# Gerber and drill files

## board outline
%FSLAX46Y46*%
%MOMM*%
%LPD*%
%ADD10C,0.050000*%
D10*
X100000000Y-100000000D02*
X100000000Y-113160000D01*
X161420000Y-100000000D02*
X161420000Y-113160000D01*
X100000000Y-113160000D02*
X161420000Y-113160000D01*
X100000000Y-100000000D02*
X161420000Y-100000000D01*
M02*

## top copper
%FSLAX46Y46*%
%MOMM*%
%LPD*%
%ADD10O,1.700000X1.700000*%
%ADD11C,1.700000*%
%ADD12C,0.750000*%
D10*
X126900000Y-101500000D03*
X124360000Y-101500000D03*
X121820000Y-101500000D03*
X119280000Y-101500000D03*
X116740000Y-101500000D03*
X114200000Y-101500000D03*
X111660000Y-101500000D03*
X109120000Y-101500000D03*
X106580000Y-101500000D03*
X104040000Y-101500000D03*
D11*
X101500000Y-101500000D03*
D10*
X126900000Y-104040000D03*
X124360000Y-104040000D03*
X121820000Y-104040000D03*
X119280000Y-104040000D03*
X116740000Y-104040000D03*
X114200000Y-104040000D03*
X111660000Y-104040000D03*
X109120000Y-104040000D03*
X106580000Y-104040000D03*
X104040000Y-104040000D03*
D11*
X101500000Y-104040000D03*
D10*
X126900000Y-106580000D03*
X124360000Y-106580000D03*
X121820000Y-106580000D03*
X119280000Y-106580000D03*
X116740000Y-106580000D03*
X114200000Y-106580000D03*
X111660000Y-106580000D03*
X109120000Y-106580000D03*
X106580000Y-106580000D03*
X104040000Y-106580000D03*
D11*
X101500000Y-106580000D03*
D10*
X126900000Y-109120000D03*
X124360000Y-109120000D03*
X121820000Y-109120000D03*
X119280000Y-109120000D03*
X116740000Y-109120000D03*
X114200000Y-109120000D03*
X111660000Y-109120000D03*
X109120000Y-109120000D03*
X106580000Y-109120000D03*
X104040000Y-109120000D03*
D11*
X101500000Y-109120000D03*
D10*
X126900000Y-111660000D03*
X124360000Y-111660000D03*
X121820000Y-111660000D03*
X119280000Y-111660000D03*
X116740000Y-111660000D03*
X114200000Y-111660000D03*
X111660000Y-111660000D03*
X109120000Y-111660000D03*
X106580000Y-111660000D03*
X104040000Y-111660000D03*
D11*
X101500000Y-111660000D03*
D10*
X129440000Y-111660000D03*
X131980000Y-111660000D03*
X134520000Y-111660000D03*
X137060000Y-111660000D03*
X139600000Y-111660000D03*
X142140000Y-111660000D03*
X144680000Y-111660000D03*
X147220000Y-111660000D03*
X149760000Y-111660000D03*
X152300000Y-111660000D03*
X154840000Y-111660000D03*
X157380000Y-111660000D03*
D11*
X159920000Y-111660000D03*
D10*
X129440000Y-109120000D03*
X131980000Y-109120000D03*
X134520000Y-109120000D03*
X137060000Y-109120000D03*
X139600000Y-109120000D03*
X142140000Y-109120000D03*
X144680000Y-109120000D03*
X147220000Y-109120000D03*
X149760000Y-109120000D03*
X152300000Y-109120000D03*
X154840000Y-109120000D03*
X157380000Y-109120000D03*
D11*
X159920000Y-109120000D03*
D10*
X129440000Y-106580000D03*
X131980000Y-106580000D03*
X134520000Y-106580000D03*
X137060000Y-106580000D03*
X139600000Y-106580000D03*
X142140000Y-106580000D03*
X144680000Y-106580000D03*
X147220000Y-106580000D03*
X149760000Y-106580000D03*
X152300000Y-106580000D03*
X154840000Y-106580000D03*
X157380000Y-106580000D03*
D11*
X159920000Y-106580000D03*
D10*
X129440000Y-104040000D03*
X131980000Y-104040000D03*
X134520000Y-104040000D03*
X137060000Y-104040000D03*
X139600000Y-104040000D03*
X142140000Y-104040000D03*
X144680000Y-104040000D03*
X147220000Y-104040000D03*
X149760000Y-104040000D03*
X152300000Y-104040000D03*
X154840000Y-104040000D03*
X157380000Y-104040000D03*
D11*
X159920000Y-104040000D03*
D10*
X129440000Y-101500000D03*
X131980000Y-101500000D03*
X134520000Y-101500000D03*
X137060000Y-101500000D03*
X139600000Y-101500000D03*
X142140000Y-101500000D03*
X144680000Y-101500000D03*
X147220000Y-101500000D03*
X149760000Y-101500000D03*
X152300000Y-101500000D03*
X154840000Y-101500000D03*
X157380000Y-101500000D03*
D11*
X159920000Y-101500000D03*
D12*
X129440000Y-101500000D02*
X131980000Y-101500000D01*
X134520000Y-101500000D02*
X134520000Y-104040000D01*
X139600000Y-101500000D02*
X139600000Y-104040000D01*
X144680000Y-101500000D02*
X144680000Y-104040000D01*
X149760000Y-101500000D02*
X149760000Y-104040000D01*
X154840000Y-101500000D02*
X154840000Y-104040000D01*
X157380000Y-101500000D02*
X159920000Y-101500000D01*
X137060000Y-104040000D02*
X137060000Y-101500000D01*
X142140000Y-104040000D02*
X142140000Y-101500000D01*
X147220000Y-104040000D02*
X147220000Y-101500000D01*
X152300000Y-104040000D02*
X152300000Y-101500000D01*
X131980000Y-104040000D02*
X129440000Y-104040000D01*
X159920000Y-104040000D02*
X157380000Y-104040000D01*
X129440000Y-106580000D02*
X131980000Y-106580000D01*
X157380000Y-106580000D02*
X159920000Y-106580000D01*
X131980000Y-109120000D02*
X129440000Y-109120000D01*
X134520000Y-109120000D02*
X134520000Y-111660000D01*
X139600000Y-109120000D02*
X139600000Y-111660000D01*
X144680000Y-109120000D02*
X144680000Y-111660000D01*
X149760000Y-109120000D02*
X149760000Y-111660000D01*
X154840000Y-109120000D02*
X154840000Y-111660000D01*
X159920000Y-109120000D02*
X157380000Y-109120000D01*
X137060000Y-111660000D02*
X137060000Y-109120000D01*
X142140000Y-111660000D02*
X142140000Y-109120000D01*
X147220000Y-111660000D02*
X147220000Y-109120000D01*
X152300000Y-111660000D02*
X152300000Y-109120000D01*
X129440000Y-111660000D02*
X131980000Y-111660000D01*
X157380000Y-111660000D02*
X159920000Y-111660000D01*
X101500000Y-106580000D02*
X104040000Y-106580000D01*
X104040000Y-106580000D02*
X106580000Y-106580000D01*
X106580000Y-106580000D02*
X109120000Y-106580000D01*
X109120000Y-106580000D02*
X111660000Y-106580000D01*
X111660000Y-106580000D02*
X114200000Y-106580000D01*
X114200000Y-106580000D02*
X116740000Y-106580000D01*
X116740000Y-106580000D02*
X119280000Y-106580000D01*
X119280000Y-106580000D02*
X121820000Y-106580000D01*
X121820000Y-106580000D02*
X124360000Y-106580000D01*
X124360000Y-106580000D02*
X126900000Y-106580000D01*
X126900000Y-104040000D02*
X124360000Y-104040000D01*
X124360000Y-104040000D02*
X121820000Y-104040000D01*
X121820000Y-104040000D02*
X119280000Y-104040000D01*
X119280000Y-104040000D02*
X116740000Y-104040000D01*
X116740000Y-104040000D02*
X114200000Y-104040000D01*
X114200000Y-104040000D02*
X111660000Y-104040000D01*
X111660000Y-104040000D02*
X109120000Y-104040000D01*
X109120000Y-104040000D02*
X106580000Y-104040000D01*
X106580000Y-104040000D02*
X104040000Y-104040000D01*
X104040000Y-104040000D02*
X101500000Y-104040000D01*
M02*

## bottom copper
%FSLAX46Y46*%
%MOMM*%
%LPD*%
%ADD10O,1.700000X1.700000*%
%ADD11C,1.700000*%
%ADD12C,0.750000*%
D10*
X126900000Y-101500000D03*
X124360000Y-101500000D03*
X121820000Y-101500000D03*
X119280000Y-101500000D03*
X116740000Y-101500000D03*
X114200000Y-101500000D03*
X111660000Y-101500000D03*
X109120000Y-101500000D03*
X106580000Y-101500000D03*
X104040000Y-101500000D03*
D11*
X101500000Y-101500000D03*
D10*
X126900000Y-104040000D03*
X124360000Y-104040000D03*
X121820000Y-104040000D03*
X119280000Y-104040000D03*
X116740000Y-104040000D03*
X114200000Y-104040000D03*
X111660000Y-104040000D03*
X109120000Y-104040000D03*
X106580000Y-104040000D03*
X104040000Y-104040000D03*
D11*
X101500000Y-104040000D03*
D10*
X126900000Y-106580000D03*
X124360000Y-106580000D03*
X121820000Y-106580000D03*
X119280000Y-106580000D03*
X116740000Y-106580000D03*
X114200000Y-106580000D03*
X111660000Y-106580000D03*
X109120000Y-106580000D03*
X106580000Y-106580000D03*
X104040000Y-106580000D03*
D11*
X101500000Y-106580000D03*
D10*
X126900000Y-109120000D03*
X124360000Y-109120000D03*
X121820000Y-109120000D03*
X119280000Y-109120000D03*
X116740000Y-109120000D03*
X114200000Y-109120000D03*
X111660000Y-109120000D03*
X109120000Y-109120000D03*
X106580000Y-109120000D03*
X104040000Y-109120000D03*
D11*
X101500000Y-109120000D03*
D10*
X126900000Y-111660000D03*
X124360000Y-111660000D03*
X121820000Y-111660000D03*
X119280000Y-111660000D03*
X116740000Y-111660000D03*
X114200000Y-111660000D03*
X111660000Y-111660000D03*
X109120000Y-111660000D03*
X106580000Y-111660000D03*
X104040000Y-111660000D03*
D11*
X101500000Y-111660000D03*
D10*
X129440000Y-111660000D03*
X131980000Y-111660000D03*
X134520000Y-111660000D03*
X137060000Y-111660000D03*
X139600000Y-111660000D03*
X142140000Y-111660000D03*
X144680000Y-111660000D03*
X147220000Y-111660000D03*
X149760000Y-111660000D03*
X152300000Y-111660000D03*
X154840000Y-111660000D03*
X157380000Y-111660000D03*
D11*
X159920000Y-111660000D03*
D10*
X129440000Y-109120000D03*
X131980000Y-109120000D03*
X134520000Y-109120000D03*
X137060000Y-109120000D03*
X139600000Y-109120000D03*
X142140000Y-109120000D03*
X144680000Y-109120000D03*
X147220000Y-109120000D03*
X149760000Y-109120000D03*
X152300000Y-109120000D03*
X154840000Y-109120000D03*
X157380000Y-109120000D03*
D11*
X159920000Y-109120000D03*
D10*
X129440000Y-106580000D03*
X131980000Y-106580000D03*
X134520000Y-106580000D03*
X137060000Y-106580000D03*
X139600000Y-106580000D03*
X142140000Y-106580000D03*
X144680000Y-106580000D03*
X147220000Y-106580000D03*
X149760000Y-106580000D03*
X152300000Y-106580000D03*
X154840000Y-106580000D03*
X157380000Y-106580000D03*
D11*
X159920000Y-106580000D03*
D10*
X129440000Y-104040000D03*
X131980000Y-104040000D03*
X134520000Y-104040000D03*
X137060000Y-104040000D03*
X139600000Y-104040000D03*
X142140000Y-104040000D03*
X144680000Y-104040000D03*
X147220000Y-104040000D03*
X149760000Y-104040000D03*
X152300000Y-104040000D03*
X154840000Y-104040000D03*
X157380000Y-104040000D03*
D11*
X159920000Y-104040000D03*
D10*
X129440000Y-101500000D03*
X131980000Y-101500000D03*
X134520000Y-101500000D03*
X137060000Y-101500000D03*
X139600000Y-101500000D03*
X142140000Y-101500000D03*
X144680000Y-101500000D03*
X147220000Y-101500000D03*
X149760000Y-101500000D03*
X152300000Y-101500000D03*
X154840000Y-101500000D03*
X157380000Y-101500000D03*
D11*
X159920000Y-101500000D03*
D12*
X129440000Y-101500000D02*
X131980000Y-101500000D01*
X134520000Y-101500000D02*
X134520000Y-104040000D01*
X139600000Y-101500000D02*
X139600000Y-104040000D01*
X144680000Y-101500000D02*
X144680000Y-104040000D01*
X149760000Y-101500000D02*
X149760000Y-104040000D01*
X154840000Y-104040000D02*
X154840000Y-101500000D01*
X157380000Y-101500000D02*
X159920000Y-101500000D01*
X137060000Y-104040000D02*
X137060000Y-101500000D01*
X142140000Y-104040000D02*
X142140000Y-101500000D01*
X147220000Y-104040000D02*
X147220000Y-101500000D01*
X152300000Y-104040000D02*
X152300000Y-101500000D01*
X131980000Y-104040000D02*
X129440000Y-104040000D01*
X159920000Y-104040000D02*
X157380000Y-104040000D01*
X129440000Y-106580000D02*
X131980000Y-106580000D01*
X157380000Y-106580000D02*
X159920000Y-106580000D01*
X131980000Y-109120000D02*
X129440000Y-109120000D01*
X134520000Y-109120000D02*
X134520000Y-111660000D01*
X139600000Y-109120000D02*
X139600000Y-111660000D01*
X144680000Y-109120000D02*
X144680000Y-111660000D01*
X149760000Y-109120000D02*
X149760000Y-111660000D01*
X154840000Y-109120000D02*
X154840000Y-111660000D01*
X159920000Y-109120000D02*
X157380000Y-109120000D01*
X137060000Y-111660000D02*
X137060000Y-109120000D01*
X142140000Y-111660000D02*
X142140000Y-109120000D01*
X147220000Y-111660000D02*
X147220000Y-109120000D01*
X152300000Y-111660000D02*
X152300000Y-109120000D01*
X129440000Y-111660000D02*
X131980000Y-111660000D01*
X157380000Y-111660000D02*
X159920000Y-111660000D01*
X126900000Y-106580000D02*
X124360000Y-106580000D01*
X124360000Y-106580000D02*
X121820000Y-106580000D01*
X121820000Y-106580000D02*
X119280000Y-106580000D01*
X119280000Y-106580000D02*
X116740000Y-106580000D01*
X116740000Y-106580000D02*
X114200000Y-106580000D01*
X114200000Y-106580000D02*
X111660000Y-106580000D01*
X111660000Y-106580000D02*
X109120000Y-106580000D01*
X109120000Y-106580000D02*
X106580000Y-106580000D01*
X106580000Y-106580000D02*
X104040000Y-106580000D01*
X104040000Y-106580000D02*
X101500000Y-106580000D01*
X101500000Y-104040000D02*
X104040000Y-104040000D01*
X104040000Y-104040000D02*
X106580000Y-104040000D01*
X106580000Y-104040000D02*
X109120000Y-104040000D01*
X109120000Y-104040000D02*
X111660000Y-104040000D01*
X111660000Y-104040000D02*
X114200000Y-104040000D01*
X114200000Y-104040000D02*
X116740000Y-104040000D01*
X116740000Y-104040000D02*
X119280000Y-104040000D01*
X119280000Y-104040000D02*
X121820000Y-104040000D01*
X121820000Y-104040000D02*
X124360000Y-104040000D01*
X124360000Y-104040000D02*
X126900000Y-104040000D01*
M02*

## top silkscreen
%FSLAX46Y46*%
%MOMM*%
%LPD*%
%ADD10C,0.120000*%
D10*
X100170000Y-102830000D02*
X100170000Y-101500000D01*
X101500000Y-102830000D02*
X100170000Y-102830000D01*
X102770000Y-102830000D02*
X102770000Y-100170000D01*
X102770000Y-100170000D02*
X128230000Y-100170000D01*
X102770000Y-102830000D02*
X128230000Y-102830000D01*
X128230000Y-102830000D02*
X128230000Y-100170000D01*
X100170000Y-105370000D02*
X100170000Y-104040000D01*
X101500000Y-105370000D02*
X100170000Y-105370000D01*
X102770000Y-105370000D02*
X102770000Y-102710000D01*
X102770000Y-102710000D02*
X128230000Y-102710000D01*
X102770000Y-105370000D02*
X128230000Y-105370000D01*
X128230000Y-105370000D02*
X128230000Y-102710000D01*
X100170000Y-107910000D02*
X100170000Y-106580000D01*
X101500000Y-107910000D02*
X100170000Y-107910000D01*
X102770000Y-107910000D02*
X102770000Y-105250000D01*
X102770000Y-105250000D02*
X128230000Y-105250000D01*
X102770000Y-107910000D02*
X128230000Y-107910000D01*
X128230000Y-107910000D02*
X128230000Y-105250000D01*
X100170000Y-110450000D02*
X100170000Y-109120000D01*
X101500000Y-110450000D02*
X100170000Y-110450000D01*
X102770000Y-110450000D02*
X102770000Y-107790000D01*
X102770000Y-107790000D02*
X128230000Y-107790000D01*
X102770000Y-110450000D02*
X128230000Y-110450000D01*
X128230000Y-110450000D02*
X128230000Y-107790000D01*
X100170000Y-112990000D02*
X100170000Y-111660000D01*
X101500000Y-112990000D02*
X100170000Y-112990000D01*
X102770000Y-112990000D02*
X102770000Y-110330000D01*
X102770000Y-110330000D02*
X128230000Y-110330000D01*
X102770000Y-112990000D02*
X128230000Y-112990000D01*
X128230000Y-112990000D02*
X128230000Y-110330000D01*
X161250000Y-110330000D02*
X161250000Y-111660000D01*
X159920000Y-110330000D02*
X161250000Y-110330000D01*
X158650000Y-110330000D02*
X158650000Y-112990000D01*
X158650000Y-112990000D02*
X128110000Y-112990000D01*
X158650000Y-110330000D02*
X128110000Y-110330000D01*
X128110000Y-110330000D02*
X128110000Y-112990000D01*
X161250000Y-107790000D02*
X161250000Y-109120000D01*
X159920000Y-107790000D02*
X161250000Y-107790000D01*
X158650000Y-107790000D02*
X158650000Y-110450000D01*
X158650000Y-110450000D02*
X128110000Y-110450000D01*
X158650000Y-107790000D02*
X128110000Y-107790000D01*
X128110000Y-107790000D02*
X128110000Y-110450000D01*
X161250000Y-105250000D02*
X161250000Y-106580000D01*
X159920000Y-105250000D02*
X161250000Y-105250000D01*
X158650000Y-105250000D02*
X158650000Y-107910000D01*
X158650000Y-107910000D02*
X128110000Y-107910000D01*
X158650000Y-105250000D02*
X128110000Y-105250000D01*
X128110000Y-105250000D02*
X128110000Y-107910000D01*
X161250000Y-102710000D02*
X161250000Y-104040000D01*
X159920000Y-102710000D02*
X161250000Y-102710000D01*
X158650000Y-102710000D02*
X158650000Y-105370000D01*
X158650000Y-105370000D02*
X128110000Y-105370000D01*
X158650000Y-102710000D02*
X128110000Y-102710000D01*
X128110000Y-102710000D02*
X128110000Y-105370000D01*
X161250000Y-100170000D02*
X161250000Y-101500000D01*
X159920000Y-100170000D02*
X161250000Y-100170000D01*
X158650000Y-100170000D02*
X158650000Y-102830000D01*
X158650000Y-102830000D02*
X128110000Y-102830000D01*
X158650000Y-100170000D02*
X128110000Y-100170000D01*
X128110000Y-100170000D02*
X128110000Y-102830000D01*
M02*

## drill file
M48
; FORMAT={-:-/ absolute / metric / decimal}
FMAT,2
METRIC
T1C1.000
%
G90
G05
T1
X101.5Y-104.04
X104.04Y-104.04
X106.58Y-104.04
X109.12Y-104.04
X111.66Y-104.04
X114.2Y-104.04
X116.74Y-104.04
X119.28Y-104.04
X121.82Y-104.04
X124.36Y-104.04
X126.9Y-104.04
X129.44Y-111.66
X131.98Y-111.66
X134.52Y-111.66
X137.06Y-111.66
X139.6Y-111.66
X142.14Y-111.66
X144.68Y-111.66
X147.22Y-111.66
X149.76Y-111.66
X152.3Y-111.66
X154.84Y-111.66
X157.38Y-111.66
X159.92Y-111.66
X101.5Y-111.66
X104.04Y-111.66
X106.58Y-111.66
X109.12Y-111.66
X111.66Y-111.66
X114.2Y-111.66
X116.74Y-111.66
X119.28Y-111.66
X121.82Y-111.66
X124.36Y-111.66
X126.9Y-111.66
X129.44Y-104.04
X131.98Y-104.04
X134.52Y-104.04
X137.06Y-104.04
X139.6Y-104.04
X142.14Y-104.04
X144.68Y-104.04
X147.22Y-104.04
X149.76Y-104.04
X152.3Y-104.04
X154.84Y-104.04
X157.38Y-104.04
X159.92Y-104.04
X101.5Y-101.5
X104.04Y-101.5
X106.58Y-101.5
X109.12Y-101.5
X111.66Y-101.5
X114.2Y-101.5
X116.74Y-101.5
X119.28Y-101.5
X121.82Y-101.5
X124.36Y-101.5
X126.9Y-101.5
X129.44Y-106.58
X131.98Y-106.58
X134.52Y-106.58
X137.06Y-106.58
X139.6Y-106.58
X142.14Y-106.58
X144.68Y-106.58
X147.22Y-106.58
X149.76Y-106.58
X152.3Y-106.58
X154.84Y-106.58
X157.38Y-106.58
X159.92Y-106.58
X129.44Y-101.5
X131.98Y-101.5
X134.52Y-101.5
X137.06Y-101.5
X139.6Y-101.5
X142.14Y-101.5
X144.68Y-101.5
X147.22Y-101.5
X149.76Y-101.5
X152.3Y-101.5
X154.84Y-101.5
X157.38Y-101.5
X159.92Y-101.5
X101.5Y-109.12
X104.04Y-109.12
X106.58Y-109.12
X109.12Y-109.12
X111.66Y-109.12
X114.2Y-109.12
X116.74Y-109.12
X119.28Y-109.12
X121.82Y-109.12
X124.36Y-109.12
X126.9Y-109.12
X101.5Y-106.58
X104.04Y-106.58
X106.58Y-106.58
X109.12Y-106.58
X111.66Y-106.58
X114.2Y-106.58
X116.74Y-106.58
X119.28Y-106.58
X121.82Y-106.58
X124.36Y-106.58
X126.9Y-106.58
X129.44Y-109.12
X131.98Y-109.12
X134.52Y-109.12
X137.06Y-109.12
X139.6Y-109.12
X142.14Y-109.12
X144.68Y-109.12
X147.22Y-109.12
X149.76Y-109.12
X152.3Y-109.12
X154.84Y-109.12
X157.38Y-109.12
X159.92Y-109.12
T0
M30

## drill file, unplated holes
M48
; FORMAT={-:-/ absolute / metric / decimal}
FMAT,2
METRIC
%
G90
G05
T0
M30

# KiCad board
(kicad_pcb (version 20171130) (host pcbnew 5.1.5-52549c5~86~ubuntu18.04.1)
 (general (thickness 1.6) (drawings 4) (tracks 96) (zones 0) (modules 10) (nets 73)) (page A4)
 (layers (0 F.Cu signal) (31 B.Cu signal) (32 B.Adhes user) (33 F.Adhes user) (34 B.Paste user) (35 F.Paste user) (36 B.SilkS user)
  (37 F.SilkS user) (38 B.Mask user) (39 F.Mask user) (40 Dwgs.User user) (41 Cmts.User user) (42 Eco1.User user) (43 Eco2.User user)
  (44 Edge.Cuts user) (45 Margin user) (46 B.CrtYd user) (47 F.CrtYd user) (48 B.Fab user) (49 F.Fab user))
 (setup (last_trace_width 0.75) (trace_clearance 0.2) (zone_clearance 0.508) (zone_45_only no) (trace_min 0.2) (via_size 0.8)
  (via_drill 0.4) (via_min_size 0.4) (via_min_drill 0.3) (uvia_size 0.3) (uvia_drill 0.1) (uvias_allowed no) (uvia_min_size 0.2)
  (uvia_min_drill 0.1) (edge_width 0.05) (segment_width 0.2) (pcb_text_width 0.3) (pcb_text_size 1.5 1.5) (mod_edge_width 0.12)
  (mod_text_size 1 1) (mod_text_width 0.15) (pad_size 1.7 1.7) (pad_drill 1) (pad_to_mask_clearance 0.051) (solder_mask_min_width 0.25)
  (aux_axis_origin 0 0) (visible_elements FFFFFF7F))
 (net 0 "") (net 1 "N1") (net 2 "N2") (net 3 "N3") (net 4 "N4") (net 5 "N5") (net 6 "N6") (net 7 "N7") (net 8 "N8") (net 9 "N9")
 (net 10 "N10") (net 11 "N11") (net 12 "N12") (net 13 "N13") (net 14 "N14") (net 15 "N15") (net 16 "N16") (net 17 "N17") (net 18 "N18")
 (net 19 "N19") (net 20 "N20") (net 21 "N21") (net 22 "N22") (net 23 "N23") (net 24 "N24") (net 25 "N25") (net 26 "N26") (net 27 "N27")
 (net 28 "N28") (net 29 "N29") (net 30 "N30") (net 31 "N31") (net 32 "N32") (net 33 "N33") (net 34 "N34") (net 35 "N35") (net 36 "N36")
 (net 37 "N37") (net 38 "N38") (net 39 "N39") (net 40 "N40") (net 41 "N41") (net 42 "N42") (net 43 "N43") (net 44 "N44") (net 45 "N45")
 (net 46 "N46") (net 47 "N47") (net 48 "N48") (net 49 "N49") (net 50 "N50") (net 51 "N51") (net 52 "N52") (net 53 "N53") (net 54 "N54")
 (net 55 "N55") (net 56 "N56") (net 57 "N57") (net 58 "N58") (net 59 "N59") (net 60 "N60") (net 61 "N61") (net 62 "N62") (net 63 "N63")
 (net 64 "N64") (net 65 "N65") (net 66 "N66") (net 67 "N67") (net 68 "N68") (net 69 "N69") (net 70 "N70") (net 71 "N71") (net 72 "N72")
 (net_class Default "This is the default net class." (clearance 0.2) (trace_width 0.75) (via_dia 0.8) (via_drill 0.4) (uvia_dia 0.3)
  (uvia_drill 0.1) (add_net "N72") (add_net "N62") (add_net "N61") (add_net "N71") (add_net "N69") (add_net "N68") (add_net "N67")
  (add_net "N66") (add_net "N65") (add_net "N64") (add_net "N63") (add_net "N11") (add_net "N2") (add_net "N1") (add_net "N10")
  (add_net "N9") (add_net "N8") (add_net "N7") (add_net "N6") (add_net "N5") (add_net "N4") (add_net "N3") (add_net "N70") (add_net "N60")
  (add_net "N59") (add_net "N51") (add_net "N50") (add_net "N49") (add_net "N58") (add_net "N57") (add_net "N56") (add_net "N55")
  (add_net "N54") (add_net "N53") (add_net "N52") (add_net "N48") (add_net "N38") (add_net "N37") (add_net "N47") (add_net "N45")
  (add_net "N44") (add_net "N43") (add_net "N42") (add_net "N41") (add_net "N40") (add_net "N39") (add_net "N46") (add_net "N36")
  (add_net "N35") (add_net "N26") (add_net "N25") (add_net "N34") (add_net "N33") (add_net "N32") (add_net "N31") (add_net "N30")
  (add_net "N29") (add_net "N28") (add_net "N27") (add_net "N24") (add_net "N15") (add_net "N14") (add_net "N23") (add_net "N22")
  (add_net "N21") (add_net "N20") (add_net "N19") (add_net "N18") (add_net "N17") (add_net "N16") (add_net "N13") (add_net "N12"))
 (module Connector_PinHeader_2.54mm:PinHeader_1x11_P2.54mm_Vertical (layer F.Cu) (at 101.5 101.5 90)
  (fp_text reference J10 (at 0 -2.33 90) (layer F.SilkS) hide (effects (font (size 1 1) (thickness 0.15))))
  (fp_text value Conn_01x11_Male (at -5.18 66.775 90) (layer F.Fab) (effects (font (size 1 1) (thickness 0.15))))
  (fp_line (start -1.33 -1.33) (end 0 -1.33) (layer F.SilkS) (width 0.12))
  (fp_line (start -1.33 0) (end -1.33 -1.33) (layer F.SilkS) (width 0.12))
  (fp_line (start -1.33 1.27) (end 1.33 1.27) (layer F.SilkS) (width 0.12))
  (fp_line (start 1.33 1.27) (end 1.33 26.73) (layer F.SilkS) (width 0.12))
  (fp_line (start -1.33 1.27) (end -1.33 26.73) (layer F.SilkS) (width 0.12))
  (fp_line (start -1.33 26.73) (end 1.33 26.73) (layer F.SilkS) (width 0.12))
  (pad 11 thru_hole oval (at 0 25.4 90) (size 1.7 1.7) (drill 1) (layers *.Cu *.Mask) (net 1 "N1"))
  (pad 10 thru_hole oval (at 0 22.86 90) (size 1.7 1.7) (drill 1) (layers *.Cu *.Mask) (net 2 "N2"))
  (pad 9 thru_hole oval (at 0 20.32 90) (size 1.7 1.7) (drill 1) (layers *.Cu *.Mask) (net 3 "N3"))
  (pad 8 thru_hole oval (at 0 17.78 90) (size 1.7 1.7) (drill 1) (layers *.Cu *.Mask) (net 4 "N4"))
  (pad 7 thru_hole oval (at 0 15.24 90) (size 1.7 1.7) (drill 1) (layers *.Cu *.Mask) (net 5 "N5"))
  (pad 6 thru_hole oval (at 0 12.7 90) (size 1.7 1.7) (drill 1) (layers *.Cu *.Mask) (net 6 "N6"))
  (pad 5 thru_hole oval (at 0 10.16 90) (size 1.7 1.7) (drill 1) (layers *.Cu *.Mask) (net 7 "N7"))
  (pad 4 thru_hole oval (at 0 7.62 90) (size 1.7 1.7) (drill 1) (layers *.Cu *.Mask) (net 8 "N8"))
  (pad 3 thru_hole oval (at 0 5.08 90) (size 1.7 1.7) (drill 1) (layers *.Cu *.Mask) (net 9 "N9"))
  (pad 2 thru_hole oval (at 0 2.54 90) (size 1.7 1.7) (drill 1) (layers *.Cu *.Mask) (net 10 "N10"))
  (pad 1 thru_hole circle (at 0 0 90) (size 1.7 1.7) (drill 1) (layers *.Cu *.Mask) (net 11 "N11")))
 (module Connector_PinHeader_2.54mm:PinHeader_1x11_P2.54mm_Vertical (layer F.Cu) (at 101.5 104.04 90)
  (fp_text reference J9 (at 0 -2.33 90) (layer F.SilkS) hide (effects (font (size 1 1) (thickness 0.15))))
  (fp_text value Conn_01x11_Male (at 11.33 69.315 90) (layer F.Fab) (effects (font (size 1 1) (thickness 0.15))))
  (fp_line (start -1.33 -1.33) (end 0 -1.33) (layer F.SilkS) (width 0.12))
  (fp_line (start -1.33 0) (end -1.33 -1.33) (layer F.SilkS) (width 0.12))
  (fp_line (start -1.33 1.27) (end 1.33 1.27) (layer F.SilkS) (width 0.12))
  (fp_line (start 1.33 1.27) (end 1.33 26.73) (layer F.SilkS) (width 0.12))
  (fp_line (start -1.33 1.27) (end -1.33 26.73) (layer F.SilkS) (width 0.12))
  (fp_line (start -1.33 26.73) (end 1.33 26.73) (layer F.SilkS) (width 0.12))
  (pad 11 thru_hole oval (at 0 25.4 90) (size 1.7 1.7) (drill 1) (layers *.Cu *.Mask) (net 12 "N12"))
  (pad 10 thru_hole oval (at 0 22.86 90) (size 1.7 1.7) (drill 1) (layers *.Cu *.Mask) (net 12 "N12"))
  (pad 9 thru_hole oval (at 0 20.32 90) (size 1.7 1.7) (drill 1) (layers *.Cu *.Mask) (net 12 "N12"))
  (pad 8 thru_hole oval (at 0 17.78 90) (size 1.7 1.7) (drill 1) (layers *.Cu *.Mask) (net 12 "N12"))
  (pad 7 thru_hole oval (at 0 15.24 90) (size 1.7 1.7) (drill 1) (layers *.Cu *.Mask) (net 12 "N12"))
  (pad 6 thru_hole oval (at 0 12.7 90) (size 1.7 1.7) (drill 1) (layers *.Cu *.Mask) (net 12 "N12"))
  (pad 5 thru_hole oval (at 0 10.16 90) (size 1.7 1.7) (drill 1) (layers *.Cu *.Mask) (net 12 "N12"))
  (pad 4 thru_hole oval (at 0 7.62 90) (size 1.7 1.7) (drill 1) (layers *.Cu *.Mask) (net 12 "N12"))
  (pad 3 thru_hole oval (at 0 5.08 90) (size 1.7 1.7) (drill 1) (layers *.Cu *.Mask) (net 12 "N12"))
  (pad 2 thru_hole oval (at 0 2.54 90) (size 1.7 1.7) (drill 1) (layers *.Cu *.Mask) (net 12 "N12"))
  (pad 1 thru_hole circle (at 0 0 90) (size 1.7 1.7) (drill 1) (layers *.Cu *.Mask) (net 12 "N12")))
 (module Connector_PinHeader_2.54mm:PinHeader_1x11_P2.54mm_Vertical (layer F.Cu) (at 101.5 106.58 90)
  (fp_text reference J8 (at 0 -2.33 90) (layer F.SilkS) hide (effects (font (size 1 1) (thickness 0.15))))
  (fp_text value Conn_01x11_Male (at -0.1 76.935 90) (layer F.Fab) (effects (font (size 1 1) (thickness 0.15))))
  (fp_line (start -1.33 -1.33) (end 0 -1.33) (layer F.SilkS) (width 0.12))
  (fp_line (start -1.33 0) (end -1.33 -1.33) (layer F.SilkS) (width 0.12))
  (fp_line (start -1.33 1.27) (end 1.33 1.27) (layer F.SilkS) (width 0.12))
  (fp_line (start 1.33 1.27) (end 1.33 26.73) (layer F.SilkS) (width 0.12))
  (fp_line (start -1.33 1.27) (end -1.33 26.73) (layer F.SilkS) (width 0.12))
  (fp_line (start -1.33 26.73) (end 1.33 26.73) (layer F.SilkS) (width 0.12))
  (pad 11 thru_hole oval (at 0 25.4 90) (size 1.7 1.7) (drill 1) (layers *.Cu *.Mask) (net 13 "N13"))
  (pad 10 thru_hole oval (at 0 22.86 90) (size 1.7 1.7) (drill 1) (layers *.Cu *.Mask) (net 13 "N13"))
  (pad 9 thru_hole oval (at 0 20.32 90) (size 1.7 1.7) (drill 1) (layers *.Cu *.Mask) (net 13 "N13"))
  (pad 8 thru_hole oval (at 0 17.78 90) (size 1.7 1.7) (drill 1) (layers *.Cu *.Mask) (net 13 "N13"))
  (pad 7 thru_hole oval (at 0 15.24 90) (size 1.7 1.7) (drill 1) (layers *.Cu *.Mask) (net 13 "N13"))
  (pad 6 thru_hole oval (at 0 12.7 90) (size 1.7 1.7) (drill 1) (layers *.Cu *.Mask) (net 13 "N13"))
  (pad 5 thru_hole oval (at 0 10.16 90) (size 1.7 1.7) (drill 1) (layers *.Cu *.Mask) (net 13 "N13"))
  (pad 4 thru_hole oval (at 0 7.62 90) (size 1.7 1.7) (drill 1) (layers *.Cu *.Mask) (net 13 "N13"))
  (pad 3 thru_hole oval (at 0 5.08 90) (size 1.7 1.7) (drill 1) (layers *.Cu *.Mask) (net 13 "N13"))
  (pad 2 thru_hole oval (at 0 2.54 90) (size 1.7 1.7) (drill 1) (layers *.Cu *.Mask) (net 13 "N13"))
  (pad 1 thru_hole circle (at 0 0 90) (size 1.7 1.7) (drill 1) (layers *.Cu *.Mask) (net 13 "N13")))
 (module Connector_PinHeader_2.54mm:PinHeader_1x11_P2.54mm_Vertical (layer F.Cu) (at 101.5 109.12 90)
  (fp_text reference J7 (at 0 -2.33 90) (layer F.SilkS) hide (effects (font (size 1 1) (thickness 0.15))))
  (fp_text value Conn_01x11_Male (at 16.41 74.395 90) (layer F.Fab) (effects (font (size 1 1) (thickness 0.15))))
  (fp_line (start -1.33 -1.33) (end 0 -1.33) (layer F.SilkS) (width 0.12))
  (fp_line (start -1.33 0) (end -1.33 -1.33) (layer F.SilkS) (width 0.12))
  (fp_line (start -1.33 1.27) (end 1.33 1.27) (layer F.SilkS) (width 0.12))
  (fp_line (start 1.33 1.27) (end 1.33 26.73) (layer F.SilkS) (width 0.12))
  (fp_line (start -1.33 1.27) (end -1.33 26.73) (layer F.SilkS) (width 0.12))
  (fp_line (start -1.33 26.73) (end 1.33 26.73) (layer F.SilkS) (width 0.12))
  (pad 11 thru_hole oval (at 0 25.4 90) (size 1.7 1.7) (drill 1) (layers *.Cu *.Mask) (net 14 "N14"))
  (pad 10 thru_hole oval (at 0 22.86 90) (size 1.7 1.7) (drill 1) (layers *.Cu *.Mask) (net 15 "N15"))
  (pad 9 thru_hole oval (at 0 20.32 90) (size 1.7 1.7) (drill 1) (layers *.Cu *.Mask) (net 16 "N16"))
  (pad 8 thru_hole oval (at 0 17.78 90) (size 1.7 1.7) (drill 1) (layers *.Cu *.Mask) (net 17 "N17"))
  (pad 7 thru_hole oval (at 0 15.24 90) (size 1.7 1.7) (drill 1) (layers *.Cu *.Mask) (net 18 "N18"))
  (pad 6 thru_hole oval (at 0 12.7 90) (size 1.7 1.7) (drill 1) (layers *.Cu *.Mask) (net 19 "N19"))
  (pad 5 thru_hole oval (at 0 10.16 90) (size 1.7 1.7) (drill 1) (layers *.Cu *.Mask) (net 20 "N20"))
  (pad 4 thru_hole oval (at 0 7.62 90) (size 1.7 1.7) (drill 1) (layers *.Cu *.Mask) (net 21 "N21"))
  (pad 3 thru_hole oval (at 0 5.08 90) (size 1.7 1.7) (drill 1) (layers *.Cu *.Mask) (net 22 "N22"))
  (pad 2 thru_hole oval (at 0 2.54 90) (size 1.7 1.7) (drill 1) (layers *.Cu *.Mask) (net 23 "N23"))
  (pad 1 thru_hole circle (at 0 0 90) (size 1.7 1.7) (drill 1) (layers *.Cu *.Mask) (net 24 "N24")))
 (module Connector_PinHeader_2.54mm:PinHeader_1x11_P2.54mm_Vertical (layer F.Cu) (at 101.5 111.66 90)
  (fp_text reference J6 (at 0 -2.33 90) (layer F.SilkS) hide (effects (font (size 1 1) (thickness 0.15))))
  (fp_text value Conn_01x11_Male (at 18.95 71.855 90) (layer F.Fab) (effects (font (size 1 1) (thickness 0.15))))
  (fp_line (start -1.33 -1.33) (end 0 -1.33) (layer F.SilkS) (width 0.12))
  (fp_line (start -1.33 0) (end -1.33 -1.33) (layer F.SilkS) (width 0.12))
  (fp_line (start -1.33 1.27) (end 1.33 1.27) (layer F.SilkS) (width 0.12))
  (fp_line (start 1.33 1.27) (end 1.33 26.73) (layer F.SilkS) (width 0.12))
  (fp_line (start -1.33 1.27) (end -1.33 26.73) (layer F.SilkS) (width 0.12))
  (fp_line (start -1.33 26.73) (end 1.33 26.73) (layer F.SilkS) (width 0.12))
  (pad 11 thru_hole oval (at 0 25.4 90) (size 1.7 1.7) (drill 1) (layers *.Cu *.Mask) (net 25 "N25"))
  (pad 10 thru_hole oval (at 0 22.86 90) (size 1.7 1.7) (drill 1) (layers *.Cu *.Mask) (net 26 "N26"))
  (pad 9 thru_hole oval (at 0 20.32 90) (size 1.7 1.7) (drill 1) (layers *.Cu *.Mask) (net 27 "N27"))
  (pad 8 thru_hole oval (at 0 17.78 90) (size 1.7 1.7) (drill 1) (layers *.Cu *.Mask) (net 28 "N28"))
  (pad 7 thru_hole oval (at 0 15.24 90) (size 1.7 1.7) (drill 1) (layers *.Cu *.Mask) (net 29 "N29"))
  (pad 6 thru_hole oval (at 0 12.7 90) (size 1.7 1.7) (drill 1) (layers *.Cu *.Mask) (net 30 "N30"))
  (pad 5 thru_hole oval (at 0 10.16 90) (size 1.7 1.7) (drill 1) (layers *.Cu *.Mask) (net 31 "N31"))
  (pad 4 thru_hole oval (at 0 7.62 90) (size 1.7 1.7) (drill 1) (layers *.Cu *.Mask) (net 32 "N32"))
  (pad 3 thru_hole oval (at 0 5.08 90) (size 1.7 1.7) (drill 1) (layers *.Cu *.Mask) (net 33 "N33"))
  (pad 2 thru_hole oval (at 0 2.54 90) (size 1.7 1.7) (drill 1) (layers *.Cu *.Mask) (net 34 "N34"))
  (pad 1 thru_hole circle (at 0 0 90) (size 1.7 1.7) (drill 1) (layers *.Cu *.Mask) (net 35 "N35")))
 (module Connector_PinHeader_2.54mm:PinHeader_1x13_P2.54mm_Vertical (layer F.Cu) (at 159.92 111.66 270)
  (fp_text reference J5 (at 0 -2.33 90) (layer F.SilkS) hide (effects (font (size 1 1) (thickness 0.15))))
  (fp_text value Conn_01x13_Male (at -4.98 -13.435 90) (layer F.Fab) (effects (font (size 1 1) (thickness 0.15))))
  (fp_line (start -1.33 -1.33) (end 0 -1.33) (layer F.SilkS) (width 0.12))
  (fp_line (start -1.33 0) (end -1.33 -1.33) (layer F.SilkS) (width 0.12))
  (fp_line (start -1.33 1.27) (end 1.33 1.27) (layer F.SilkS) (width 0.12))
  (fp_line (start 1.33 1.27) (end 1.33 31.81) (layer F.SilkS) (width 0.12))
  (fp_line (start -1.33 1.27) (end -1.33 31.81) (layer F.SilkS) (width 0.12))
  (fp_line (start -1.33 31.81) (end 1.33 31.81) (layer F.SilkS) (width 0.12))
  (pad 13 thru_hole oval (at 0 30.48 270) (size 1.7 1.7) (drill 1) (layers *.Cu *.Mask) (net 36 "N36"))
  (pad 12 thru_hole oval (at 0 27.94 270) (size 1.7 1.7) (drill 1) (layers *.Cu *.Mask) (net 36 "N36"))
  (pad 11 thru_hole oval (at 0 25.4 270) (size 1.7 1.7) (drill 1) (layers *.Cu *.Mask) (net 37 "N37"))
  (pad 10 thru_hole oval (at 0 22.86 270) (size 1.7 1.7) (drill 1) (layers *.Cu *.Mask) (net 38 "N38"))
  (pad 9 thru_hole oval (at 0 20.32 270) (size 1.7 1.7) (drill 1) (layers *.Cu *.Mask) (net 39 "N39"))
  (pad 8 thru_hole oval (at 0 17.78 270) (size 1.7 1.7) (drill 1) (layers *.Cu *.Mask) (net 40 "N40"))
  (pad 7 thru_hole oval (at 0 15.24 270) (size 1.7 1.7) (drill 1) (layers *.Cu *.Mask) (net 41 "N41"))
  (pad 6 thru_hole oval (at 0 12.7 270) (size 1.7 1.7) (drill 1) (layers *.Cu *.Mask) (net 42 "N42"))
  (pad 5 thru_hole oval (at 0 10.16 270) (size 1.7 1.7) (drill 1) (layers *.Cu *.Mask) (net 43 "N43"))
  (pad 4 thru_hole oval (at 0 7.62 270) (size 1.7 1.7) (drill 1) (layers *.Cu *.Mask) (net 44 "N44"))
  (pad 3 thru_hole oval (at 0 5.08 270) (size 1.7 1.7) (drill 1) (layers *.Cu *.Mask) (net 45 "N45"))
  (pad 2 thru_hole oval (at 0 2.54 270) (size 1.7 1.7) (drill 1) (layers *.Cu *.Mask) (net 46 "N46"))
  (pad 1 thru_hole circle (at 0 0 270) (size 1.7 1.7) (drill 1) (layers *.Cu *.Mask) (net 46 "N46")))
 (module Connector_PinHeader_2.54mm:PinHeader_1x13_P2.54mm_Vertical (layer F.Cu) (at 159.92 109.12 270)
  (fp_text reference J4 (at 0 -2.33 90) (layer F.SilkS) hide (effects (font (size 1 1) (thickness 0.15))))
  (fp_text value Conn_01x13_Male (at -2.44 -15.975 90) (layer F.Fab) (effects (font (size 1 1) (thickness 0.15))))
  (fp_line (start -1.33 -1.33) (end 0 -1.33) (layer F.SilkS) (width 0.12))
  (fp_line (start -1.33 0) (end -1.33 -1.33) (layer F.SilkS) (width 0.12))
  (fp_line (start -1.33 1.27) (end 1.33 1.27) (layer F.SilkS) (width 0.12))
  (fp_line (start 1.33 1.27) (end 1.33 31.81) (layer F.SilkS) (width 0.12))
  (fp_line (start -1.33 1.27) (end -1.33 31.81) (layer F.SilkS) (width 0.12))
  (fp_line (start -1.33 31.81) (end 1.33 31.81) (layer F.SilkS) (width 0.12))
  (pad 13 thru_hole oval (at 0 30.48 270) (size 1.7 1.7) (drill 1) (layers *.Cu *.Mask) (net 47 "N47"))
  (pad 12 thru_hole oval (at 0 27.94 270) (size 1.7 1.7) (drill 1) (layers *.Cu *.Mask) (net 47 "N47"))
  (pad 11 thru_hole oval (at 0 25.4 270) (size 1.7 1.7) (drill 1) (layers *.Cu *.Mask) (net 37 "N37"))
  (pad 10 thru_hole oval (at 0 22.86 270) (size 1.7 1.7) (drill 1) (layers *.Cu *.Mask) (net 38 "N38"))
  (pad 9 thru_hole oval (at 0 20.32 270) (size 1.7 1.7) (drill 1) (layers *.Cu *.Mask) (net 39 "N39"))
  (pad 8 thru_hole oval (at 0 17.78 270) (size 1.7 1.7) (drill 1) (layers *.Cu *.Mask) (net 40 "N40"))
  (pad 7 thru_hole oval (at 0 15.24 270) (size 1.7 1.7) (drill 1) (layers *.Cu *.Mask) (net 41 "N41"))
  (pad 6 thru_hole oval (at 0 12.7 270) (size 1.7 1.7) (drill 1) (layers *.Cu *.Mask) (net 42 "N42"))
  (pad 5 thru_hole oval (at 0 10.16 270) (size 1.7 1.7) (drill 1) (layers *.Cu *.Mask) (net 43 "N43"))
  (pad 4 thru_hole oval (at 0 7.62 270) (size 1.7 1.7) (drill 1) (layers *.Cu *.Mask) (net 44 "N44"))
  (pad 3 thru_hole oval (at 0 5.08 270) (size 1.7 1.7) (drill 1) (layers *.Cu *.Mask) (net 45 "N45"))
  (pad 2 thru_hole oval (at 0 2.54 270) (size 1.7 1.7) (drill 1) (layers *.Cu *.Mask) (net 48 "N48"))
  (pad 1 thru_hole circle (at 0 0 270) (size 1.7 1.7) (drill 1) (layers *.Cu *.Mask) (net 48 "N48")))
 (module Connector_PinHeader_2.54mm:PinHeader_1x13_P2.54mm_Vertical (layer F.Cu) (at 159.92 106.58 270)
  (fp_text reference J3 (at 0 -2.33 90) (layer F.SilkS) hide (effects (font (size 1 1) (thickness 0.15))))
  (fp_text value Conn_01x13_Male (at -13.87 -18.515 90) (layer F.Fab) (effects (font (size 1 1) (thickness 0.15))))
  (fp_line (start -1.33 -1.33) (end 0 -1.33) (layer F.SilkS) (width 0.12))
  (fp_line (start -1.33 0) (end -1.33 -1.33) (layer F.SilkS) (width 0.12))
  (fp_line (start -1.33 1.27) (end 1.33 1.27) (layer F.SilkS) (width 0.12))
  (fp_line (start 1.33 1.27) (end 1.33 31.81) (layer F.SilkS) (width 0.12))
  (fp_line (start -1.33 1.27) (end -1.33 31.81) (layer F.SilkS) (width 0.12))
  (fp_line (start -1.33 31.81) (end 1.33 31.81) (layer F.SilkS) (width 0.12))
  (pad 13 thru_hole oval (at 0 30.48 270) (size 1.7 1.7) (drill 1) (layers *.Cu *.Mask) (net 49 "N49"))
  (pad 12 thru_hole oval (at 0 27.94 270) (size 1.7 1.7) (drill 1) (layers *.Cu *.Mask) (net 49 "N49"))
  (pad 11 thru_hole oval (at 0 25.4 270) (size 1.7 1.7) (drill 1) (layers *.Cu *.Mask) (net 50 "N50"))
  (pad 10 thru_hole oval (at 0 22.86 270) (size 1.7 1.7) (drill 1) (layers *.Cu *.Mask) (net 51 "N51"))
  (pad 9 thru_hole oval (at 0 20.32 270) (size 1.7 1.7) (drill 1) (layers *.Cu *.Mask) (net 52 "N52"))
  (pad 8 thru_hole oval (at 0 17.78 270) (size 1.7 1.7) (drill 1) (layers *.Cu *.Mask) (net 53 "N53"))
  (pad 7 thru_hole oval (at 0 15.24 270) (size 1.7 1.7) (drill 1) (layers *.Cu *.Mask) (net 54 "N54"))
  (pad 6 thru_hole oval (at 0 12.7 270) (size 1.7 1.7) (drill 1) (layers *.Cu *.Mask) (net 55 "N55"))
  (pad 5 thru_hole oval (at 0 10.16 270) (size 1.7 1.7) (drill 1) (layers *.Cu *.Mask) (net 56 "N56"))
  (pad 4 thru_hole oval (at 0 7.62 270) (size 1.7 1.7) (drill 1) (layers *.Cu *.Mask) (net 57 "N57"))
  (pad 3 thru_hole oval (at 0 5.08 270) (size 1.7 1.7) (drill 1) (layers *.Cu *.Mask) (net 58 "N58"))
  (pad 2 thru_hole oval (at 0 2.54 270) (size 1.7 1.7) (drill 1) (layers *.Cu *.Mask) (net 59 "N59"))
  (pad 1 thru_hole circle (at 0 0 270) (size 1.7 1.7) (drill 1) (layers *.Cu *.Mask) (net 59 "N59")))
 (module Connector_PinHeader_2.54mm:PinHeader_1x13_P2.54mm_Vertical (layer F.Cu) (at 159.92 104.04 270)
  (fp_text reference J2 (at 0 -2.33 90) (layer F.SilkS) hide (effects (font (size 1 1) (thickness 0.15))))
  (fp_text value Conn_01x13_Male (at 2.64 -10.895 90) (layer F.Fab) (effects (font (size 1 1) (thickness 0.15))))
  (fp_line (start -1.33 -1.33) (end 0 -1.33) (layer F.SilkS) (width 0.12))
  (fp_line (start -1.33 0) (end -1.33 -1.33) (layer F.SilkS) (width 0.12))
  (fp_line (start -1.33 1.27) (end 1.33 1.27) (layer F.SilkS) (width 0.12))
  (fp_line (start 1.33 1.27) (end 1.33 31.81) (layer F.SilkS) (width 0.12))
  (fp_line (start -1.33 1.27) (end -1.33 31.81) (layer F.SilkS) (width 0.12))
  (fp_line (start -1.33 31.81) (end 1.33 31.81) (layer F.SilkS) (width 0.12))
  (pad 13 thru_hole oval (at 0 30.48 270) (size 1.7 1.7) (drill 1) (layers *.Cu *.Mask) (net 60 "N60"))
  (pad 12 thru_hole oval (at 0 27.94 270) (size 1.7 1.7) (drill 1) (layers *.Cu *.Mask) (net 60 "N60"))
  (pad 11 thru_hole oval (at 0 25.4 270) (size 1.7 1.7) (drill 1) (layers *.Cu *.Mask) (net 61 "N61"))
  (pad 10 thru_hole oval (at 0 22.86 270) (size 1.7 1.7) (drill 1) (layers *.Cu *.Mask) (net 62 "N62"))
  (pad 9 thru_hole oval (at 0 20.32 270) (size 1.7 1.7) (drill 1) (layers *.Cu *.Mask) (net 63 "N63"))
  (pad 8 thru_hole oval (at 0 17.78 270) (size 1.7 1.7) (drill 1) (layers *.Cu *.Mask) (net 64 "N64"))
  (pad 7 thru_hole oval (at 0 15.24 270) (size 1.7 1.7) (drill 1) (layers *.Cu *.Mask) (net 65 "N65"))
  (pad 6 thru_hole oval (at 0 12.7 270) (size 1.7 1.7) (drill 1) (layers *.Cu *.Mask) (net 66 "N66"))
  (pad 5 thru_hole oval (at 0 10.16 270) (size 1.7 1.7) (drill 1) (layers *.Cu *.Mask) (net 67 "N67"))
  (pad 4 thru_hole oval (at 0 7.62 270) (size 1.7 1.7) (drill 1) (layers *.Cu *.Mask) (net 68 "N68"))
  (pad 3 thru_hole oval (at 0 5.08 270) (size 1.7 1.7) (drill 1) (layers *.Cu *.Mask) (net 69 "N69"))
  (pad 2 thru_hole oval (at 0 2.54 270) (size 1.7 1.7) (drill 1) (layers *.Cu *.Mask) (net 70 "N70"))
  (pad 1 thru_hole circle (at 0 0 270) (size 1.7 1.7) (drill 1) (layers *.Cu *.Mask) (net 70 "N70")))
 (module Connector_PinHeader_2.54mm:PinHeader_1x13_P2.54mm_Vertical (layer F.Cu) (at 159.92 101.5 270)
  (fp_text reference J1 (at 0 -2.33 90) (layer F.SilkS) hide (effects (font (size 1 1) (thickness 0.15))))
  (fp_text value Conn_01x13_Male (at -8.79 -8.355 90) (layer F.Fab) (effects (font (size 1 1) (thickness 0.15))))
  (fp_line (start -1.33 -1.33) (end 0 -1.33) (layer F.SilkS) (width 0.12))
  (fp_line (start -1.33 0) (end -1.33 -1.33) (layer F.SilkS) (width 0.12))
  (fp_line (start -1.33 1.27) (end 1.33 1.27) (layer F.SilkS) (width 0.12))
  (fp_line (start 1.33 1.27) (end 1.33 31.81) (layer F.SilkS) (width 0.12))
  (fp_line (start -1.33 1.27) (end -1.33 31.81) (layer F.SilkS) (width 0.12))
  (fp_line (start -1.33 31.81) (end 1.33 31.81) (layer F.SilkS) (width 0.12))
  (pad 13 thru_hole oval (at 0 30.48 270) (size 1.7 1.7) (drill 1) (layers *.Cu *.Mask) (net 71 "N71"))
  (pad 12 thru_hole oval (at 0 27.94 270) (size 1.7 1.7) (drill 1) (layers *.Cu *.Mask) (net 71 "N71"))
  (pad 11 thru_hole oval (at 0 25.4 270) (size 1.7 1.7) (drill 1) (layers *.Cu *.Mask) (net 61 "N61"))
  (pad 10 thru_hole oval (at 0 22.86 270) (size 1.7 1.7) (drill 1) (layers *.Cu *.Mask) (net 62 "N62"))
  (pad 9 thru_hole oval (at 0 20.32 270) (size 1.7 1.7) (drill 1) (layers *.Cu *.Mask) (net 63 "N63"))
  (pad 8 thru_hole oval (at 0 17.78 270) (size 1.7 1.7) (drill 1) (layers *.Cu *.Mask) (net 64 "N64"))
  (pad 7 thru_hole oval (at 0 15.24 270) (size 1.7 1.7) (drill 1) (layers *.Cu *.Mask) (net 65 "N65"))
  (pad 6 thru_hole oval (at 0 12.7 270) (size 1.7 1.7) (drill 1) (layers *.Cu *.Mask) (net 66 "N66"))
  (pad 5 thru_hole oval (at 0 10.16 270) (size 1.7 1.7) (drill 1) (layers *.Cu *.Mask) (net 67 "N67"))
  (pad 4 thru_hole oval (at 0 7.62 270) (size 1.7 1.7) (drill 1) (layers *.Cu *.Mask) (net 68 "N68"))
  (pad 3 thru_hole oval (at 0 5.08 270) (size 1.7 1.7) (drill 1) (layers *.Cu *.Mask) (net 69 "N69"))
  (pad 2 thru_hole oval (at 0 2.54 270) (size 1.7 1.7) (drill 1) (layers *.Cu *.Mask) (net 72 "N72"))
  (pad 1 thru_hole circle (at 0 0 270) (size 1.7 1.7) (drill 1) (layers *.Cu *.Mask) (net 72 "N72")))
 (gr_line (start 100 100) (end 100 113.16) (layer Edge.Cuts) (width 0.05))
 (gr_line (start 161.42 100) (end 161.42 113.16) (layer Edge.Cuts) (width 0.05))
 (gr_line (start 100 113.16) (end 161.42 113.16) (layer Edge.Cuts) (width 0.05))
 (gr_line (start 100 100) (end 161.42 100) (layer Edge.Cuts) (width 0.05))
 (segment (start 129.44 101.5) (end 131.98 101.5) (width 0.75) (layer B.Cu) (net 71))
 (segment (start 129.44 101.5) (end 131.98 101.5) (width 0.75) (layer F.Cu) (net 71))
 (segment (start 134.52 101.5) (end 134.52 104.04) (width 0.75) (layer B.Cu) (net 61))
 (segment (start 134.52 101.5) (end 134.52 104.04) (width 0.75) (layer F.Cu) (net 61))
 (segment (start 139.6 101.5) (end 139.6 104.04) (width 0.75) (layer B.Cu) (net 63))
 (segment (start 139.6 101.5) (end 139.6 104.04) (width 0.75) (layer F.Cu) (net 63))
 (segment (start 144.68 101.5) (end 144.68 104.04) (width 0.75) (layer B.Cu) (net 65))
 (segment (start 144.68 101.5) (end 144.68 104.04) (width 0.75) (layer F.Cu) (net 65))
 (segment (start 149.76 101.5) (end 149.76 104.04) (width 0.75) (layer B.Cu) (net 67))
 (segment (start 149.76 101.5) (end 149.76 104.04) (width 0.75) (layer F.Cu) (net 67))
 (segment (start 154.84 104.04) (end 154.84 101.5) (width 0.75) (layer B.Cu) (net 69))
 (segment (start 154.84 101.5) (end 154.84 104.04) (width 0.75) (layer F.Cu) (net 69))
 (segment (start 157.38 101.5) (end 159.92 101.5) (width 0.75) (layer B.Cu) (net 72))
 (segment (start 157.38 101.5) (end 159.92 101.5) (width 0.75) (layer F.Cu) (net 72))
 (segment (start 137.06 104.04) (end 137.06 101.5) (width 0.75) (layer B.Cu) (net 62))
 (segment (start 137.06 104.04) (end 137.06 101.5) (width 0.75) (layer F.Cu) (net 62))
 (segment (start 142.14 104.04) (end 142.14 101.5) (width 0.75) (layer B.Cu) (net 64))
 (segment (start 142.14 104.04) (end 142.14 101.5) (width 0.75) (layer F.Cu) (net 64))
 (segment (start 147.22 104.04) (end 147.22 101.5) (width 0.75) (layer B.Cu) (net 66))
 (segment (start 147.22 104.04) (end 147.22 101.5) (width 0.75) (layer F.Cu) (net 66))
 (segment (start 152.3 104.04) (end 152.3 101.5) (width 0.75) (layer B.Cu) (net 68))
 (segment (start 152.3 104.04) (end 152.3 101.5) (width 0.75) (layer F.Cu) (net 68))
 (segment (start 131.98 104.04) (end 129.44 104.04) (width 0.75) (layer B.Cu) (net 60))
 (segment (start 131.98 104.04) (end 129.44 104.04) (width 0.75) (layer F.Cu) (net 60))
 (segment (start 159.92 104.04) (end 157.38 104.04) (width 0.75) (layer B.Cu) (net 70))
 (segment (start 159.92 104.04) (end 157.38 104.04) (width 0.75) (layer F.Cu) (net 70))
 (segment (start 129.44 106.58) (end 131.98 106.58) (width 0.75) (layer B.Cu) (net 49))
 (segment (start 129.44 106.58) (end 131.98 106.58) (width 0.75) (layer F.Cu) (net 49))
 (segment (start 157.38 106.58) (end 159.92 106.58) (width 0.75) (layer B.Cu) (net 59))
 (segment (start 157.38 106.58) (end 159.92 106.58) (width 0.75) (layer F.Cu) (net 59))
 (segment (start 131.98 109.12) (end 129.44 109.12) (width 0.75) (layer B.Cu) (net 47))
 (segment (start 131.98 109.12) (end 129.44 109.12) (width 0.75) (layer F.Cu) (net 47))
 (segment (start 134.52 109.12) (end 134.52 111.66) (width 0.75) (layer B.Cu) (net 37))
 (segment (start 134.52 109.12) (end 134.52 111.66) (width 0.75) (layer F.Cu) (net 37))
 (segment (start 139.6 109.12) (end 139.6 111.66) (width 0.75) (layer B.Cu) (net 39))
 (segment (start 139.6 109.12) (end 139.6 111.66) (width 0.75) (layer F.Cu) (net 39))
 (segment (start 144.68 109.12) (end 144.68 111.66) (width 0.75) (layer B.Cu) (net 41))
 (segment (start 144.68 109.12) (end 144.68 111.66) (width 0.75) (layer F.Cu) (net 41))
 (segment (start 149.76 109.12) (end 149.76 111.66) (width 0.75) (layer B.Cu) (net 43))
 (segment (start 149.76 109.12) (end 149.76 111.66) (width 0.75) (layer F.Cu) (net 43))
 (segment (start 154.84 109.12) (end 154.84 111.66) (width 0.75) (layer B.Cu) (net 45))
 (segment (start 154.84 109.12) (end 154.84 111.66) (width 0.75) (layer F.Cu) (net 45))
 (segment (start 159.92 109.12) (end 157.38 109.12) (width 0.75) (layer B.Cu) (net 48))
 (segment (start 159.92 109.12) (end 157.38 109.12) (width 0.75) (layer F.Cu) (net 48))
 (segment (start 137.06 111.66) (end 137.06 109.12) (width 0.75) (layer B.Cu) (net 38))
 (segment (start 137.06 111.66) (end 137.06 109.12) (width 0.75) (layer F.Cu) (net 38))
 (segment (start 142.14 111.66) (end 142.14 109.12) (width 0.75) (layer B.Cu) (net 40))
 (segment (start 142.14 111.66) (end 142.14 109.12) (width 0.75) (layer F.Cu) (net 40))
 (segment (start 147.22 111.66) (end 147.22 109.12) (width 0.75) (layer B.Cu) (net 42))
 (segment (start 147.22 111.66) (end 147.22 109.12) (width 0.75) (layer F.Cu) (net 42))
 (segment (start 152.3 111.66) (end 152.3 109.12) (width 0.75) (layer B.Cu) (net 44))
 (segment (start 152.3 111.66) (end 152.3 109.12) (width 0.75) (layer F.Cu) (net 44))
 (segment (start 129.44 111.66) (end 131.98 111.66) (width 0.75) (layer B.Cu) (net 36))
 (segment (start 129.44 111.66) (end 131.98 111.66) (width 0.75) (layer F.Cu) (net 36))
 (segment (start 157.38 111.66) (end 159.92 111.66) (width 0.75) (layer B.Cu) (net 46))
 (segment (start 157.38 111.66) (end 159.92 111.66) (width 0.75) (layer F.Cu) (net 46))
 (segment (start 126.9 106.58) (end 124.36 106.58) (width 0.75) (layer B.Cu) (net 13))
 (segment (start 124.36 106.58) (end 121.82 106.58) (width 0.75) (layer B.Cu) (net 13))
 (segment (start 121.82 106.58) (end 119.28 106.58) (width 0.75) (layer B.Cu) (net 13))
 (segment (start 119.28 106.58) (end 116.74 106.58) (width 0.75) (layer B.Cu) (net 13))
 (segment (start 116.74 106.58) (end 114.2 106.58) (width 0.75) (layer B.Cu) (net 13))
 (segment (start 114.2 106.58) (end 111.66 106.58) (width 0.75) (layer B.Cu) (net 13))
 (segment (start 111.66 106.58) (end 109.12 106.58) (width 0.75) (layer B.Cu) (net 13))
 (segment (start 109.12 106.58) (end 106.58 106.58) (width 0.75) (layer B.Cu) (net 13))
 (segment (start 106.58 106.58) (end 104.04 106.58) (width 0.75) (layer B.Cu) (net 13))
 (segment (start 104.04 106.58) (end 101.5 106.58) (width 0.75) (layer B.Cu) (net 13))
 (segment (start 101.5 106.58) (end 104.04 106.58) (width 0.75) (layer F.Cu) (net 13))
 (segment (start 104.04 106.58) (end 106.58 106.58) (width 0.75) (layer F.Cu) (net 13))
 (segment (start 106.58 106.58) (end 109.12 106.58) (width 0.75) (layer F.Cu) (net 13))
 (segment (start 109.12 106.58) (end 111.66 106.58) (width 0.75) (layer F.Cu) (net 13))
 (segment (start 111.66 106.58) (end 114.2 106.58) (width 0.75) (layer F.Cu) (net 13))
 (segment (start 114.2 106.58) (end 116.74 106.58) (width 0.75) (layer F.Cu) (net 13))
 (segment (start 116.74 106.58) (end 119.28 106.58) (width 0.75) (layer F.Cu) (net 13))
 (segment (start 119.28 106.58) (end 121.82 106.58) (width 0.75) (layer F.Cu) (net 13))
 (segment (start 121.82 106.58) (end 124.36 106.58) (width 0.75) (layer F.Cu) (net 13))
 (segment (start 124.36 106.58) (end 126.9 106.58) (width 0.75) (layer F.Cu) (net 13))
 (segment (start 101.5 104.04) (end 104.04 104.04) (width 0.75) (layer B.Cu) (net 12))
 (segment (start 104.04 104.04) (end 106.58 104.04) (width 0.75) (layer B.Cu) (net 12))
 (segment (start 106.58 104.04) (end 109.12 104.04) (width 0.75) (layer B.Cu) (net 12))
 (segment (start 109.12 104.04) (end 111.66 104.04) (width 0.75) (layer B.Cu) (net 12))
 (segment (start 111.66 104.04) (end 114.2 104.04) (width 0.75) (layer B.Cu) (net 12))
 (segment (start 114.2 104.04) (end 116.74 104.04) (width 0.75) (layer B.Cu) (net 12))
 (segment (start 116.74 104.04) (end 119.28 104.04) (width 0.75) (layer B.Cu) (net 12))
 (segment (start 119.28 104.04) (end 121.82 104.04) (width 0.75) (layer B.Cu) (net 12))
 (segment (start 121.82 104.04) (end 124.36 104.04) (width 0.75) (layer B.Cu) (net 12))
 (segment (start 124.36 104.04) (end 126.9 104.04) (width 0.75) (layer B.Cu) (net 12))
 (segment (start 126.9 104.04) (end 124.36 104.04) (width 0.75) (layer F.Cu) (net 12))
 (segment (start 124.36 104.04) (end 121.82 104.04) (width 0.75) (layer F.Cu) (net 12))
 (segment (start 121.82 104.04) (end 119.28 104.04) (width 0.75) (layer F.Cu) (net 12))
 (segment (start 119.28 104.04) (end 116.74 104.04) (width 0.75) (layer F.Cu) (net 12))
 (segment (start 116.74 104.04) (end 114.2 104.04) (width 0.75) (layer F.Cu) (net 12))
 (segment (start 114.2 104.04) (end 111.66 104.04) (width 0.75) (layer F.Cu) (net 12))
 (segment (start 111.66 104.04) (end 109.12 104.04) (width 0.75) (layer F.Cu) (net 12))
 (segment (start 109.12 104.04) (end 106.58 104.04) (width 0.75) (layer F.Cu) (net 12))
 (segment (start 106.58 104.04) (end 104.04 104.04) (width 0.75) (layer F.Cu) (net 12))
 (segment (start 104.04 104.04) (end 101.5 104.04) (width 0.75) (layer F.Cu) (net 12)))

